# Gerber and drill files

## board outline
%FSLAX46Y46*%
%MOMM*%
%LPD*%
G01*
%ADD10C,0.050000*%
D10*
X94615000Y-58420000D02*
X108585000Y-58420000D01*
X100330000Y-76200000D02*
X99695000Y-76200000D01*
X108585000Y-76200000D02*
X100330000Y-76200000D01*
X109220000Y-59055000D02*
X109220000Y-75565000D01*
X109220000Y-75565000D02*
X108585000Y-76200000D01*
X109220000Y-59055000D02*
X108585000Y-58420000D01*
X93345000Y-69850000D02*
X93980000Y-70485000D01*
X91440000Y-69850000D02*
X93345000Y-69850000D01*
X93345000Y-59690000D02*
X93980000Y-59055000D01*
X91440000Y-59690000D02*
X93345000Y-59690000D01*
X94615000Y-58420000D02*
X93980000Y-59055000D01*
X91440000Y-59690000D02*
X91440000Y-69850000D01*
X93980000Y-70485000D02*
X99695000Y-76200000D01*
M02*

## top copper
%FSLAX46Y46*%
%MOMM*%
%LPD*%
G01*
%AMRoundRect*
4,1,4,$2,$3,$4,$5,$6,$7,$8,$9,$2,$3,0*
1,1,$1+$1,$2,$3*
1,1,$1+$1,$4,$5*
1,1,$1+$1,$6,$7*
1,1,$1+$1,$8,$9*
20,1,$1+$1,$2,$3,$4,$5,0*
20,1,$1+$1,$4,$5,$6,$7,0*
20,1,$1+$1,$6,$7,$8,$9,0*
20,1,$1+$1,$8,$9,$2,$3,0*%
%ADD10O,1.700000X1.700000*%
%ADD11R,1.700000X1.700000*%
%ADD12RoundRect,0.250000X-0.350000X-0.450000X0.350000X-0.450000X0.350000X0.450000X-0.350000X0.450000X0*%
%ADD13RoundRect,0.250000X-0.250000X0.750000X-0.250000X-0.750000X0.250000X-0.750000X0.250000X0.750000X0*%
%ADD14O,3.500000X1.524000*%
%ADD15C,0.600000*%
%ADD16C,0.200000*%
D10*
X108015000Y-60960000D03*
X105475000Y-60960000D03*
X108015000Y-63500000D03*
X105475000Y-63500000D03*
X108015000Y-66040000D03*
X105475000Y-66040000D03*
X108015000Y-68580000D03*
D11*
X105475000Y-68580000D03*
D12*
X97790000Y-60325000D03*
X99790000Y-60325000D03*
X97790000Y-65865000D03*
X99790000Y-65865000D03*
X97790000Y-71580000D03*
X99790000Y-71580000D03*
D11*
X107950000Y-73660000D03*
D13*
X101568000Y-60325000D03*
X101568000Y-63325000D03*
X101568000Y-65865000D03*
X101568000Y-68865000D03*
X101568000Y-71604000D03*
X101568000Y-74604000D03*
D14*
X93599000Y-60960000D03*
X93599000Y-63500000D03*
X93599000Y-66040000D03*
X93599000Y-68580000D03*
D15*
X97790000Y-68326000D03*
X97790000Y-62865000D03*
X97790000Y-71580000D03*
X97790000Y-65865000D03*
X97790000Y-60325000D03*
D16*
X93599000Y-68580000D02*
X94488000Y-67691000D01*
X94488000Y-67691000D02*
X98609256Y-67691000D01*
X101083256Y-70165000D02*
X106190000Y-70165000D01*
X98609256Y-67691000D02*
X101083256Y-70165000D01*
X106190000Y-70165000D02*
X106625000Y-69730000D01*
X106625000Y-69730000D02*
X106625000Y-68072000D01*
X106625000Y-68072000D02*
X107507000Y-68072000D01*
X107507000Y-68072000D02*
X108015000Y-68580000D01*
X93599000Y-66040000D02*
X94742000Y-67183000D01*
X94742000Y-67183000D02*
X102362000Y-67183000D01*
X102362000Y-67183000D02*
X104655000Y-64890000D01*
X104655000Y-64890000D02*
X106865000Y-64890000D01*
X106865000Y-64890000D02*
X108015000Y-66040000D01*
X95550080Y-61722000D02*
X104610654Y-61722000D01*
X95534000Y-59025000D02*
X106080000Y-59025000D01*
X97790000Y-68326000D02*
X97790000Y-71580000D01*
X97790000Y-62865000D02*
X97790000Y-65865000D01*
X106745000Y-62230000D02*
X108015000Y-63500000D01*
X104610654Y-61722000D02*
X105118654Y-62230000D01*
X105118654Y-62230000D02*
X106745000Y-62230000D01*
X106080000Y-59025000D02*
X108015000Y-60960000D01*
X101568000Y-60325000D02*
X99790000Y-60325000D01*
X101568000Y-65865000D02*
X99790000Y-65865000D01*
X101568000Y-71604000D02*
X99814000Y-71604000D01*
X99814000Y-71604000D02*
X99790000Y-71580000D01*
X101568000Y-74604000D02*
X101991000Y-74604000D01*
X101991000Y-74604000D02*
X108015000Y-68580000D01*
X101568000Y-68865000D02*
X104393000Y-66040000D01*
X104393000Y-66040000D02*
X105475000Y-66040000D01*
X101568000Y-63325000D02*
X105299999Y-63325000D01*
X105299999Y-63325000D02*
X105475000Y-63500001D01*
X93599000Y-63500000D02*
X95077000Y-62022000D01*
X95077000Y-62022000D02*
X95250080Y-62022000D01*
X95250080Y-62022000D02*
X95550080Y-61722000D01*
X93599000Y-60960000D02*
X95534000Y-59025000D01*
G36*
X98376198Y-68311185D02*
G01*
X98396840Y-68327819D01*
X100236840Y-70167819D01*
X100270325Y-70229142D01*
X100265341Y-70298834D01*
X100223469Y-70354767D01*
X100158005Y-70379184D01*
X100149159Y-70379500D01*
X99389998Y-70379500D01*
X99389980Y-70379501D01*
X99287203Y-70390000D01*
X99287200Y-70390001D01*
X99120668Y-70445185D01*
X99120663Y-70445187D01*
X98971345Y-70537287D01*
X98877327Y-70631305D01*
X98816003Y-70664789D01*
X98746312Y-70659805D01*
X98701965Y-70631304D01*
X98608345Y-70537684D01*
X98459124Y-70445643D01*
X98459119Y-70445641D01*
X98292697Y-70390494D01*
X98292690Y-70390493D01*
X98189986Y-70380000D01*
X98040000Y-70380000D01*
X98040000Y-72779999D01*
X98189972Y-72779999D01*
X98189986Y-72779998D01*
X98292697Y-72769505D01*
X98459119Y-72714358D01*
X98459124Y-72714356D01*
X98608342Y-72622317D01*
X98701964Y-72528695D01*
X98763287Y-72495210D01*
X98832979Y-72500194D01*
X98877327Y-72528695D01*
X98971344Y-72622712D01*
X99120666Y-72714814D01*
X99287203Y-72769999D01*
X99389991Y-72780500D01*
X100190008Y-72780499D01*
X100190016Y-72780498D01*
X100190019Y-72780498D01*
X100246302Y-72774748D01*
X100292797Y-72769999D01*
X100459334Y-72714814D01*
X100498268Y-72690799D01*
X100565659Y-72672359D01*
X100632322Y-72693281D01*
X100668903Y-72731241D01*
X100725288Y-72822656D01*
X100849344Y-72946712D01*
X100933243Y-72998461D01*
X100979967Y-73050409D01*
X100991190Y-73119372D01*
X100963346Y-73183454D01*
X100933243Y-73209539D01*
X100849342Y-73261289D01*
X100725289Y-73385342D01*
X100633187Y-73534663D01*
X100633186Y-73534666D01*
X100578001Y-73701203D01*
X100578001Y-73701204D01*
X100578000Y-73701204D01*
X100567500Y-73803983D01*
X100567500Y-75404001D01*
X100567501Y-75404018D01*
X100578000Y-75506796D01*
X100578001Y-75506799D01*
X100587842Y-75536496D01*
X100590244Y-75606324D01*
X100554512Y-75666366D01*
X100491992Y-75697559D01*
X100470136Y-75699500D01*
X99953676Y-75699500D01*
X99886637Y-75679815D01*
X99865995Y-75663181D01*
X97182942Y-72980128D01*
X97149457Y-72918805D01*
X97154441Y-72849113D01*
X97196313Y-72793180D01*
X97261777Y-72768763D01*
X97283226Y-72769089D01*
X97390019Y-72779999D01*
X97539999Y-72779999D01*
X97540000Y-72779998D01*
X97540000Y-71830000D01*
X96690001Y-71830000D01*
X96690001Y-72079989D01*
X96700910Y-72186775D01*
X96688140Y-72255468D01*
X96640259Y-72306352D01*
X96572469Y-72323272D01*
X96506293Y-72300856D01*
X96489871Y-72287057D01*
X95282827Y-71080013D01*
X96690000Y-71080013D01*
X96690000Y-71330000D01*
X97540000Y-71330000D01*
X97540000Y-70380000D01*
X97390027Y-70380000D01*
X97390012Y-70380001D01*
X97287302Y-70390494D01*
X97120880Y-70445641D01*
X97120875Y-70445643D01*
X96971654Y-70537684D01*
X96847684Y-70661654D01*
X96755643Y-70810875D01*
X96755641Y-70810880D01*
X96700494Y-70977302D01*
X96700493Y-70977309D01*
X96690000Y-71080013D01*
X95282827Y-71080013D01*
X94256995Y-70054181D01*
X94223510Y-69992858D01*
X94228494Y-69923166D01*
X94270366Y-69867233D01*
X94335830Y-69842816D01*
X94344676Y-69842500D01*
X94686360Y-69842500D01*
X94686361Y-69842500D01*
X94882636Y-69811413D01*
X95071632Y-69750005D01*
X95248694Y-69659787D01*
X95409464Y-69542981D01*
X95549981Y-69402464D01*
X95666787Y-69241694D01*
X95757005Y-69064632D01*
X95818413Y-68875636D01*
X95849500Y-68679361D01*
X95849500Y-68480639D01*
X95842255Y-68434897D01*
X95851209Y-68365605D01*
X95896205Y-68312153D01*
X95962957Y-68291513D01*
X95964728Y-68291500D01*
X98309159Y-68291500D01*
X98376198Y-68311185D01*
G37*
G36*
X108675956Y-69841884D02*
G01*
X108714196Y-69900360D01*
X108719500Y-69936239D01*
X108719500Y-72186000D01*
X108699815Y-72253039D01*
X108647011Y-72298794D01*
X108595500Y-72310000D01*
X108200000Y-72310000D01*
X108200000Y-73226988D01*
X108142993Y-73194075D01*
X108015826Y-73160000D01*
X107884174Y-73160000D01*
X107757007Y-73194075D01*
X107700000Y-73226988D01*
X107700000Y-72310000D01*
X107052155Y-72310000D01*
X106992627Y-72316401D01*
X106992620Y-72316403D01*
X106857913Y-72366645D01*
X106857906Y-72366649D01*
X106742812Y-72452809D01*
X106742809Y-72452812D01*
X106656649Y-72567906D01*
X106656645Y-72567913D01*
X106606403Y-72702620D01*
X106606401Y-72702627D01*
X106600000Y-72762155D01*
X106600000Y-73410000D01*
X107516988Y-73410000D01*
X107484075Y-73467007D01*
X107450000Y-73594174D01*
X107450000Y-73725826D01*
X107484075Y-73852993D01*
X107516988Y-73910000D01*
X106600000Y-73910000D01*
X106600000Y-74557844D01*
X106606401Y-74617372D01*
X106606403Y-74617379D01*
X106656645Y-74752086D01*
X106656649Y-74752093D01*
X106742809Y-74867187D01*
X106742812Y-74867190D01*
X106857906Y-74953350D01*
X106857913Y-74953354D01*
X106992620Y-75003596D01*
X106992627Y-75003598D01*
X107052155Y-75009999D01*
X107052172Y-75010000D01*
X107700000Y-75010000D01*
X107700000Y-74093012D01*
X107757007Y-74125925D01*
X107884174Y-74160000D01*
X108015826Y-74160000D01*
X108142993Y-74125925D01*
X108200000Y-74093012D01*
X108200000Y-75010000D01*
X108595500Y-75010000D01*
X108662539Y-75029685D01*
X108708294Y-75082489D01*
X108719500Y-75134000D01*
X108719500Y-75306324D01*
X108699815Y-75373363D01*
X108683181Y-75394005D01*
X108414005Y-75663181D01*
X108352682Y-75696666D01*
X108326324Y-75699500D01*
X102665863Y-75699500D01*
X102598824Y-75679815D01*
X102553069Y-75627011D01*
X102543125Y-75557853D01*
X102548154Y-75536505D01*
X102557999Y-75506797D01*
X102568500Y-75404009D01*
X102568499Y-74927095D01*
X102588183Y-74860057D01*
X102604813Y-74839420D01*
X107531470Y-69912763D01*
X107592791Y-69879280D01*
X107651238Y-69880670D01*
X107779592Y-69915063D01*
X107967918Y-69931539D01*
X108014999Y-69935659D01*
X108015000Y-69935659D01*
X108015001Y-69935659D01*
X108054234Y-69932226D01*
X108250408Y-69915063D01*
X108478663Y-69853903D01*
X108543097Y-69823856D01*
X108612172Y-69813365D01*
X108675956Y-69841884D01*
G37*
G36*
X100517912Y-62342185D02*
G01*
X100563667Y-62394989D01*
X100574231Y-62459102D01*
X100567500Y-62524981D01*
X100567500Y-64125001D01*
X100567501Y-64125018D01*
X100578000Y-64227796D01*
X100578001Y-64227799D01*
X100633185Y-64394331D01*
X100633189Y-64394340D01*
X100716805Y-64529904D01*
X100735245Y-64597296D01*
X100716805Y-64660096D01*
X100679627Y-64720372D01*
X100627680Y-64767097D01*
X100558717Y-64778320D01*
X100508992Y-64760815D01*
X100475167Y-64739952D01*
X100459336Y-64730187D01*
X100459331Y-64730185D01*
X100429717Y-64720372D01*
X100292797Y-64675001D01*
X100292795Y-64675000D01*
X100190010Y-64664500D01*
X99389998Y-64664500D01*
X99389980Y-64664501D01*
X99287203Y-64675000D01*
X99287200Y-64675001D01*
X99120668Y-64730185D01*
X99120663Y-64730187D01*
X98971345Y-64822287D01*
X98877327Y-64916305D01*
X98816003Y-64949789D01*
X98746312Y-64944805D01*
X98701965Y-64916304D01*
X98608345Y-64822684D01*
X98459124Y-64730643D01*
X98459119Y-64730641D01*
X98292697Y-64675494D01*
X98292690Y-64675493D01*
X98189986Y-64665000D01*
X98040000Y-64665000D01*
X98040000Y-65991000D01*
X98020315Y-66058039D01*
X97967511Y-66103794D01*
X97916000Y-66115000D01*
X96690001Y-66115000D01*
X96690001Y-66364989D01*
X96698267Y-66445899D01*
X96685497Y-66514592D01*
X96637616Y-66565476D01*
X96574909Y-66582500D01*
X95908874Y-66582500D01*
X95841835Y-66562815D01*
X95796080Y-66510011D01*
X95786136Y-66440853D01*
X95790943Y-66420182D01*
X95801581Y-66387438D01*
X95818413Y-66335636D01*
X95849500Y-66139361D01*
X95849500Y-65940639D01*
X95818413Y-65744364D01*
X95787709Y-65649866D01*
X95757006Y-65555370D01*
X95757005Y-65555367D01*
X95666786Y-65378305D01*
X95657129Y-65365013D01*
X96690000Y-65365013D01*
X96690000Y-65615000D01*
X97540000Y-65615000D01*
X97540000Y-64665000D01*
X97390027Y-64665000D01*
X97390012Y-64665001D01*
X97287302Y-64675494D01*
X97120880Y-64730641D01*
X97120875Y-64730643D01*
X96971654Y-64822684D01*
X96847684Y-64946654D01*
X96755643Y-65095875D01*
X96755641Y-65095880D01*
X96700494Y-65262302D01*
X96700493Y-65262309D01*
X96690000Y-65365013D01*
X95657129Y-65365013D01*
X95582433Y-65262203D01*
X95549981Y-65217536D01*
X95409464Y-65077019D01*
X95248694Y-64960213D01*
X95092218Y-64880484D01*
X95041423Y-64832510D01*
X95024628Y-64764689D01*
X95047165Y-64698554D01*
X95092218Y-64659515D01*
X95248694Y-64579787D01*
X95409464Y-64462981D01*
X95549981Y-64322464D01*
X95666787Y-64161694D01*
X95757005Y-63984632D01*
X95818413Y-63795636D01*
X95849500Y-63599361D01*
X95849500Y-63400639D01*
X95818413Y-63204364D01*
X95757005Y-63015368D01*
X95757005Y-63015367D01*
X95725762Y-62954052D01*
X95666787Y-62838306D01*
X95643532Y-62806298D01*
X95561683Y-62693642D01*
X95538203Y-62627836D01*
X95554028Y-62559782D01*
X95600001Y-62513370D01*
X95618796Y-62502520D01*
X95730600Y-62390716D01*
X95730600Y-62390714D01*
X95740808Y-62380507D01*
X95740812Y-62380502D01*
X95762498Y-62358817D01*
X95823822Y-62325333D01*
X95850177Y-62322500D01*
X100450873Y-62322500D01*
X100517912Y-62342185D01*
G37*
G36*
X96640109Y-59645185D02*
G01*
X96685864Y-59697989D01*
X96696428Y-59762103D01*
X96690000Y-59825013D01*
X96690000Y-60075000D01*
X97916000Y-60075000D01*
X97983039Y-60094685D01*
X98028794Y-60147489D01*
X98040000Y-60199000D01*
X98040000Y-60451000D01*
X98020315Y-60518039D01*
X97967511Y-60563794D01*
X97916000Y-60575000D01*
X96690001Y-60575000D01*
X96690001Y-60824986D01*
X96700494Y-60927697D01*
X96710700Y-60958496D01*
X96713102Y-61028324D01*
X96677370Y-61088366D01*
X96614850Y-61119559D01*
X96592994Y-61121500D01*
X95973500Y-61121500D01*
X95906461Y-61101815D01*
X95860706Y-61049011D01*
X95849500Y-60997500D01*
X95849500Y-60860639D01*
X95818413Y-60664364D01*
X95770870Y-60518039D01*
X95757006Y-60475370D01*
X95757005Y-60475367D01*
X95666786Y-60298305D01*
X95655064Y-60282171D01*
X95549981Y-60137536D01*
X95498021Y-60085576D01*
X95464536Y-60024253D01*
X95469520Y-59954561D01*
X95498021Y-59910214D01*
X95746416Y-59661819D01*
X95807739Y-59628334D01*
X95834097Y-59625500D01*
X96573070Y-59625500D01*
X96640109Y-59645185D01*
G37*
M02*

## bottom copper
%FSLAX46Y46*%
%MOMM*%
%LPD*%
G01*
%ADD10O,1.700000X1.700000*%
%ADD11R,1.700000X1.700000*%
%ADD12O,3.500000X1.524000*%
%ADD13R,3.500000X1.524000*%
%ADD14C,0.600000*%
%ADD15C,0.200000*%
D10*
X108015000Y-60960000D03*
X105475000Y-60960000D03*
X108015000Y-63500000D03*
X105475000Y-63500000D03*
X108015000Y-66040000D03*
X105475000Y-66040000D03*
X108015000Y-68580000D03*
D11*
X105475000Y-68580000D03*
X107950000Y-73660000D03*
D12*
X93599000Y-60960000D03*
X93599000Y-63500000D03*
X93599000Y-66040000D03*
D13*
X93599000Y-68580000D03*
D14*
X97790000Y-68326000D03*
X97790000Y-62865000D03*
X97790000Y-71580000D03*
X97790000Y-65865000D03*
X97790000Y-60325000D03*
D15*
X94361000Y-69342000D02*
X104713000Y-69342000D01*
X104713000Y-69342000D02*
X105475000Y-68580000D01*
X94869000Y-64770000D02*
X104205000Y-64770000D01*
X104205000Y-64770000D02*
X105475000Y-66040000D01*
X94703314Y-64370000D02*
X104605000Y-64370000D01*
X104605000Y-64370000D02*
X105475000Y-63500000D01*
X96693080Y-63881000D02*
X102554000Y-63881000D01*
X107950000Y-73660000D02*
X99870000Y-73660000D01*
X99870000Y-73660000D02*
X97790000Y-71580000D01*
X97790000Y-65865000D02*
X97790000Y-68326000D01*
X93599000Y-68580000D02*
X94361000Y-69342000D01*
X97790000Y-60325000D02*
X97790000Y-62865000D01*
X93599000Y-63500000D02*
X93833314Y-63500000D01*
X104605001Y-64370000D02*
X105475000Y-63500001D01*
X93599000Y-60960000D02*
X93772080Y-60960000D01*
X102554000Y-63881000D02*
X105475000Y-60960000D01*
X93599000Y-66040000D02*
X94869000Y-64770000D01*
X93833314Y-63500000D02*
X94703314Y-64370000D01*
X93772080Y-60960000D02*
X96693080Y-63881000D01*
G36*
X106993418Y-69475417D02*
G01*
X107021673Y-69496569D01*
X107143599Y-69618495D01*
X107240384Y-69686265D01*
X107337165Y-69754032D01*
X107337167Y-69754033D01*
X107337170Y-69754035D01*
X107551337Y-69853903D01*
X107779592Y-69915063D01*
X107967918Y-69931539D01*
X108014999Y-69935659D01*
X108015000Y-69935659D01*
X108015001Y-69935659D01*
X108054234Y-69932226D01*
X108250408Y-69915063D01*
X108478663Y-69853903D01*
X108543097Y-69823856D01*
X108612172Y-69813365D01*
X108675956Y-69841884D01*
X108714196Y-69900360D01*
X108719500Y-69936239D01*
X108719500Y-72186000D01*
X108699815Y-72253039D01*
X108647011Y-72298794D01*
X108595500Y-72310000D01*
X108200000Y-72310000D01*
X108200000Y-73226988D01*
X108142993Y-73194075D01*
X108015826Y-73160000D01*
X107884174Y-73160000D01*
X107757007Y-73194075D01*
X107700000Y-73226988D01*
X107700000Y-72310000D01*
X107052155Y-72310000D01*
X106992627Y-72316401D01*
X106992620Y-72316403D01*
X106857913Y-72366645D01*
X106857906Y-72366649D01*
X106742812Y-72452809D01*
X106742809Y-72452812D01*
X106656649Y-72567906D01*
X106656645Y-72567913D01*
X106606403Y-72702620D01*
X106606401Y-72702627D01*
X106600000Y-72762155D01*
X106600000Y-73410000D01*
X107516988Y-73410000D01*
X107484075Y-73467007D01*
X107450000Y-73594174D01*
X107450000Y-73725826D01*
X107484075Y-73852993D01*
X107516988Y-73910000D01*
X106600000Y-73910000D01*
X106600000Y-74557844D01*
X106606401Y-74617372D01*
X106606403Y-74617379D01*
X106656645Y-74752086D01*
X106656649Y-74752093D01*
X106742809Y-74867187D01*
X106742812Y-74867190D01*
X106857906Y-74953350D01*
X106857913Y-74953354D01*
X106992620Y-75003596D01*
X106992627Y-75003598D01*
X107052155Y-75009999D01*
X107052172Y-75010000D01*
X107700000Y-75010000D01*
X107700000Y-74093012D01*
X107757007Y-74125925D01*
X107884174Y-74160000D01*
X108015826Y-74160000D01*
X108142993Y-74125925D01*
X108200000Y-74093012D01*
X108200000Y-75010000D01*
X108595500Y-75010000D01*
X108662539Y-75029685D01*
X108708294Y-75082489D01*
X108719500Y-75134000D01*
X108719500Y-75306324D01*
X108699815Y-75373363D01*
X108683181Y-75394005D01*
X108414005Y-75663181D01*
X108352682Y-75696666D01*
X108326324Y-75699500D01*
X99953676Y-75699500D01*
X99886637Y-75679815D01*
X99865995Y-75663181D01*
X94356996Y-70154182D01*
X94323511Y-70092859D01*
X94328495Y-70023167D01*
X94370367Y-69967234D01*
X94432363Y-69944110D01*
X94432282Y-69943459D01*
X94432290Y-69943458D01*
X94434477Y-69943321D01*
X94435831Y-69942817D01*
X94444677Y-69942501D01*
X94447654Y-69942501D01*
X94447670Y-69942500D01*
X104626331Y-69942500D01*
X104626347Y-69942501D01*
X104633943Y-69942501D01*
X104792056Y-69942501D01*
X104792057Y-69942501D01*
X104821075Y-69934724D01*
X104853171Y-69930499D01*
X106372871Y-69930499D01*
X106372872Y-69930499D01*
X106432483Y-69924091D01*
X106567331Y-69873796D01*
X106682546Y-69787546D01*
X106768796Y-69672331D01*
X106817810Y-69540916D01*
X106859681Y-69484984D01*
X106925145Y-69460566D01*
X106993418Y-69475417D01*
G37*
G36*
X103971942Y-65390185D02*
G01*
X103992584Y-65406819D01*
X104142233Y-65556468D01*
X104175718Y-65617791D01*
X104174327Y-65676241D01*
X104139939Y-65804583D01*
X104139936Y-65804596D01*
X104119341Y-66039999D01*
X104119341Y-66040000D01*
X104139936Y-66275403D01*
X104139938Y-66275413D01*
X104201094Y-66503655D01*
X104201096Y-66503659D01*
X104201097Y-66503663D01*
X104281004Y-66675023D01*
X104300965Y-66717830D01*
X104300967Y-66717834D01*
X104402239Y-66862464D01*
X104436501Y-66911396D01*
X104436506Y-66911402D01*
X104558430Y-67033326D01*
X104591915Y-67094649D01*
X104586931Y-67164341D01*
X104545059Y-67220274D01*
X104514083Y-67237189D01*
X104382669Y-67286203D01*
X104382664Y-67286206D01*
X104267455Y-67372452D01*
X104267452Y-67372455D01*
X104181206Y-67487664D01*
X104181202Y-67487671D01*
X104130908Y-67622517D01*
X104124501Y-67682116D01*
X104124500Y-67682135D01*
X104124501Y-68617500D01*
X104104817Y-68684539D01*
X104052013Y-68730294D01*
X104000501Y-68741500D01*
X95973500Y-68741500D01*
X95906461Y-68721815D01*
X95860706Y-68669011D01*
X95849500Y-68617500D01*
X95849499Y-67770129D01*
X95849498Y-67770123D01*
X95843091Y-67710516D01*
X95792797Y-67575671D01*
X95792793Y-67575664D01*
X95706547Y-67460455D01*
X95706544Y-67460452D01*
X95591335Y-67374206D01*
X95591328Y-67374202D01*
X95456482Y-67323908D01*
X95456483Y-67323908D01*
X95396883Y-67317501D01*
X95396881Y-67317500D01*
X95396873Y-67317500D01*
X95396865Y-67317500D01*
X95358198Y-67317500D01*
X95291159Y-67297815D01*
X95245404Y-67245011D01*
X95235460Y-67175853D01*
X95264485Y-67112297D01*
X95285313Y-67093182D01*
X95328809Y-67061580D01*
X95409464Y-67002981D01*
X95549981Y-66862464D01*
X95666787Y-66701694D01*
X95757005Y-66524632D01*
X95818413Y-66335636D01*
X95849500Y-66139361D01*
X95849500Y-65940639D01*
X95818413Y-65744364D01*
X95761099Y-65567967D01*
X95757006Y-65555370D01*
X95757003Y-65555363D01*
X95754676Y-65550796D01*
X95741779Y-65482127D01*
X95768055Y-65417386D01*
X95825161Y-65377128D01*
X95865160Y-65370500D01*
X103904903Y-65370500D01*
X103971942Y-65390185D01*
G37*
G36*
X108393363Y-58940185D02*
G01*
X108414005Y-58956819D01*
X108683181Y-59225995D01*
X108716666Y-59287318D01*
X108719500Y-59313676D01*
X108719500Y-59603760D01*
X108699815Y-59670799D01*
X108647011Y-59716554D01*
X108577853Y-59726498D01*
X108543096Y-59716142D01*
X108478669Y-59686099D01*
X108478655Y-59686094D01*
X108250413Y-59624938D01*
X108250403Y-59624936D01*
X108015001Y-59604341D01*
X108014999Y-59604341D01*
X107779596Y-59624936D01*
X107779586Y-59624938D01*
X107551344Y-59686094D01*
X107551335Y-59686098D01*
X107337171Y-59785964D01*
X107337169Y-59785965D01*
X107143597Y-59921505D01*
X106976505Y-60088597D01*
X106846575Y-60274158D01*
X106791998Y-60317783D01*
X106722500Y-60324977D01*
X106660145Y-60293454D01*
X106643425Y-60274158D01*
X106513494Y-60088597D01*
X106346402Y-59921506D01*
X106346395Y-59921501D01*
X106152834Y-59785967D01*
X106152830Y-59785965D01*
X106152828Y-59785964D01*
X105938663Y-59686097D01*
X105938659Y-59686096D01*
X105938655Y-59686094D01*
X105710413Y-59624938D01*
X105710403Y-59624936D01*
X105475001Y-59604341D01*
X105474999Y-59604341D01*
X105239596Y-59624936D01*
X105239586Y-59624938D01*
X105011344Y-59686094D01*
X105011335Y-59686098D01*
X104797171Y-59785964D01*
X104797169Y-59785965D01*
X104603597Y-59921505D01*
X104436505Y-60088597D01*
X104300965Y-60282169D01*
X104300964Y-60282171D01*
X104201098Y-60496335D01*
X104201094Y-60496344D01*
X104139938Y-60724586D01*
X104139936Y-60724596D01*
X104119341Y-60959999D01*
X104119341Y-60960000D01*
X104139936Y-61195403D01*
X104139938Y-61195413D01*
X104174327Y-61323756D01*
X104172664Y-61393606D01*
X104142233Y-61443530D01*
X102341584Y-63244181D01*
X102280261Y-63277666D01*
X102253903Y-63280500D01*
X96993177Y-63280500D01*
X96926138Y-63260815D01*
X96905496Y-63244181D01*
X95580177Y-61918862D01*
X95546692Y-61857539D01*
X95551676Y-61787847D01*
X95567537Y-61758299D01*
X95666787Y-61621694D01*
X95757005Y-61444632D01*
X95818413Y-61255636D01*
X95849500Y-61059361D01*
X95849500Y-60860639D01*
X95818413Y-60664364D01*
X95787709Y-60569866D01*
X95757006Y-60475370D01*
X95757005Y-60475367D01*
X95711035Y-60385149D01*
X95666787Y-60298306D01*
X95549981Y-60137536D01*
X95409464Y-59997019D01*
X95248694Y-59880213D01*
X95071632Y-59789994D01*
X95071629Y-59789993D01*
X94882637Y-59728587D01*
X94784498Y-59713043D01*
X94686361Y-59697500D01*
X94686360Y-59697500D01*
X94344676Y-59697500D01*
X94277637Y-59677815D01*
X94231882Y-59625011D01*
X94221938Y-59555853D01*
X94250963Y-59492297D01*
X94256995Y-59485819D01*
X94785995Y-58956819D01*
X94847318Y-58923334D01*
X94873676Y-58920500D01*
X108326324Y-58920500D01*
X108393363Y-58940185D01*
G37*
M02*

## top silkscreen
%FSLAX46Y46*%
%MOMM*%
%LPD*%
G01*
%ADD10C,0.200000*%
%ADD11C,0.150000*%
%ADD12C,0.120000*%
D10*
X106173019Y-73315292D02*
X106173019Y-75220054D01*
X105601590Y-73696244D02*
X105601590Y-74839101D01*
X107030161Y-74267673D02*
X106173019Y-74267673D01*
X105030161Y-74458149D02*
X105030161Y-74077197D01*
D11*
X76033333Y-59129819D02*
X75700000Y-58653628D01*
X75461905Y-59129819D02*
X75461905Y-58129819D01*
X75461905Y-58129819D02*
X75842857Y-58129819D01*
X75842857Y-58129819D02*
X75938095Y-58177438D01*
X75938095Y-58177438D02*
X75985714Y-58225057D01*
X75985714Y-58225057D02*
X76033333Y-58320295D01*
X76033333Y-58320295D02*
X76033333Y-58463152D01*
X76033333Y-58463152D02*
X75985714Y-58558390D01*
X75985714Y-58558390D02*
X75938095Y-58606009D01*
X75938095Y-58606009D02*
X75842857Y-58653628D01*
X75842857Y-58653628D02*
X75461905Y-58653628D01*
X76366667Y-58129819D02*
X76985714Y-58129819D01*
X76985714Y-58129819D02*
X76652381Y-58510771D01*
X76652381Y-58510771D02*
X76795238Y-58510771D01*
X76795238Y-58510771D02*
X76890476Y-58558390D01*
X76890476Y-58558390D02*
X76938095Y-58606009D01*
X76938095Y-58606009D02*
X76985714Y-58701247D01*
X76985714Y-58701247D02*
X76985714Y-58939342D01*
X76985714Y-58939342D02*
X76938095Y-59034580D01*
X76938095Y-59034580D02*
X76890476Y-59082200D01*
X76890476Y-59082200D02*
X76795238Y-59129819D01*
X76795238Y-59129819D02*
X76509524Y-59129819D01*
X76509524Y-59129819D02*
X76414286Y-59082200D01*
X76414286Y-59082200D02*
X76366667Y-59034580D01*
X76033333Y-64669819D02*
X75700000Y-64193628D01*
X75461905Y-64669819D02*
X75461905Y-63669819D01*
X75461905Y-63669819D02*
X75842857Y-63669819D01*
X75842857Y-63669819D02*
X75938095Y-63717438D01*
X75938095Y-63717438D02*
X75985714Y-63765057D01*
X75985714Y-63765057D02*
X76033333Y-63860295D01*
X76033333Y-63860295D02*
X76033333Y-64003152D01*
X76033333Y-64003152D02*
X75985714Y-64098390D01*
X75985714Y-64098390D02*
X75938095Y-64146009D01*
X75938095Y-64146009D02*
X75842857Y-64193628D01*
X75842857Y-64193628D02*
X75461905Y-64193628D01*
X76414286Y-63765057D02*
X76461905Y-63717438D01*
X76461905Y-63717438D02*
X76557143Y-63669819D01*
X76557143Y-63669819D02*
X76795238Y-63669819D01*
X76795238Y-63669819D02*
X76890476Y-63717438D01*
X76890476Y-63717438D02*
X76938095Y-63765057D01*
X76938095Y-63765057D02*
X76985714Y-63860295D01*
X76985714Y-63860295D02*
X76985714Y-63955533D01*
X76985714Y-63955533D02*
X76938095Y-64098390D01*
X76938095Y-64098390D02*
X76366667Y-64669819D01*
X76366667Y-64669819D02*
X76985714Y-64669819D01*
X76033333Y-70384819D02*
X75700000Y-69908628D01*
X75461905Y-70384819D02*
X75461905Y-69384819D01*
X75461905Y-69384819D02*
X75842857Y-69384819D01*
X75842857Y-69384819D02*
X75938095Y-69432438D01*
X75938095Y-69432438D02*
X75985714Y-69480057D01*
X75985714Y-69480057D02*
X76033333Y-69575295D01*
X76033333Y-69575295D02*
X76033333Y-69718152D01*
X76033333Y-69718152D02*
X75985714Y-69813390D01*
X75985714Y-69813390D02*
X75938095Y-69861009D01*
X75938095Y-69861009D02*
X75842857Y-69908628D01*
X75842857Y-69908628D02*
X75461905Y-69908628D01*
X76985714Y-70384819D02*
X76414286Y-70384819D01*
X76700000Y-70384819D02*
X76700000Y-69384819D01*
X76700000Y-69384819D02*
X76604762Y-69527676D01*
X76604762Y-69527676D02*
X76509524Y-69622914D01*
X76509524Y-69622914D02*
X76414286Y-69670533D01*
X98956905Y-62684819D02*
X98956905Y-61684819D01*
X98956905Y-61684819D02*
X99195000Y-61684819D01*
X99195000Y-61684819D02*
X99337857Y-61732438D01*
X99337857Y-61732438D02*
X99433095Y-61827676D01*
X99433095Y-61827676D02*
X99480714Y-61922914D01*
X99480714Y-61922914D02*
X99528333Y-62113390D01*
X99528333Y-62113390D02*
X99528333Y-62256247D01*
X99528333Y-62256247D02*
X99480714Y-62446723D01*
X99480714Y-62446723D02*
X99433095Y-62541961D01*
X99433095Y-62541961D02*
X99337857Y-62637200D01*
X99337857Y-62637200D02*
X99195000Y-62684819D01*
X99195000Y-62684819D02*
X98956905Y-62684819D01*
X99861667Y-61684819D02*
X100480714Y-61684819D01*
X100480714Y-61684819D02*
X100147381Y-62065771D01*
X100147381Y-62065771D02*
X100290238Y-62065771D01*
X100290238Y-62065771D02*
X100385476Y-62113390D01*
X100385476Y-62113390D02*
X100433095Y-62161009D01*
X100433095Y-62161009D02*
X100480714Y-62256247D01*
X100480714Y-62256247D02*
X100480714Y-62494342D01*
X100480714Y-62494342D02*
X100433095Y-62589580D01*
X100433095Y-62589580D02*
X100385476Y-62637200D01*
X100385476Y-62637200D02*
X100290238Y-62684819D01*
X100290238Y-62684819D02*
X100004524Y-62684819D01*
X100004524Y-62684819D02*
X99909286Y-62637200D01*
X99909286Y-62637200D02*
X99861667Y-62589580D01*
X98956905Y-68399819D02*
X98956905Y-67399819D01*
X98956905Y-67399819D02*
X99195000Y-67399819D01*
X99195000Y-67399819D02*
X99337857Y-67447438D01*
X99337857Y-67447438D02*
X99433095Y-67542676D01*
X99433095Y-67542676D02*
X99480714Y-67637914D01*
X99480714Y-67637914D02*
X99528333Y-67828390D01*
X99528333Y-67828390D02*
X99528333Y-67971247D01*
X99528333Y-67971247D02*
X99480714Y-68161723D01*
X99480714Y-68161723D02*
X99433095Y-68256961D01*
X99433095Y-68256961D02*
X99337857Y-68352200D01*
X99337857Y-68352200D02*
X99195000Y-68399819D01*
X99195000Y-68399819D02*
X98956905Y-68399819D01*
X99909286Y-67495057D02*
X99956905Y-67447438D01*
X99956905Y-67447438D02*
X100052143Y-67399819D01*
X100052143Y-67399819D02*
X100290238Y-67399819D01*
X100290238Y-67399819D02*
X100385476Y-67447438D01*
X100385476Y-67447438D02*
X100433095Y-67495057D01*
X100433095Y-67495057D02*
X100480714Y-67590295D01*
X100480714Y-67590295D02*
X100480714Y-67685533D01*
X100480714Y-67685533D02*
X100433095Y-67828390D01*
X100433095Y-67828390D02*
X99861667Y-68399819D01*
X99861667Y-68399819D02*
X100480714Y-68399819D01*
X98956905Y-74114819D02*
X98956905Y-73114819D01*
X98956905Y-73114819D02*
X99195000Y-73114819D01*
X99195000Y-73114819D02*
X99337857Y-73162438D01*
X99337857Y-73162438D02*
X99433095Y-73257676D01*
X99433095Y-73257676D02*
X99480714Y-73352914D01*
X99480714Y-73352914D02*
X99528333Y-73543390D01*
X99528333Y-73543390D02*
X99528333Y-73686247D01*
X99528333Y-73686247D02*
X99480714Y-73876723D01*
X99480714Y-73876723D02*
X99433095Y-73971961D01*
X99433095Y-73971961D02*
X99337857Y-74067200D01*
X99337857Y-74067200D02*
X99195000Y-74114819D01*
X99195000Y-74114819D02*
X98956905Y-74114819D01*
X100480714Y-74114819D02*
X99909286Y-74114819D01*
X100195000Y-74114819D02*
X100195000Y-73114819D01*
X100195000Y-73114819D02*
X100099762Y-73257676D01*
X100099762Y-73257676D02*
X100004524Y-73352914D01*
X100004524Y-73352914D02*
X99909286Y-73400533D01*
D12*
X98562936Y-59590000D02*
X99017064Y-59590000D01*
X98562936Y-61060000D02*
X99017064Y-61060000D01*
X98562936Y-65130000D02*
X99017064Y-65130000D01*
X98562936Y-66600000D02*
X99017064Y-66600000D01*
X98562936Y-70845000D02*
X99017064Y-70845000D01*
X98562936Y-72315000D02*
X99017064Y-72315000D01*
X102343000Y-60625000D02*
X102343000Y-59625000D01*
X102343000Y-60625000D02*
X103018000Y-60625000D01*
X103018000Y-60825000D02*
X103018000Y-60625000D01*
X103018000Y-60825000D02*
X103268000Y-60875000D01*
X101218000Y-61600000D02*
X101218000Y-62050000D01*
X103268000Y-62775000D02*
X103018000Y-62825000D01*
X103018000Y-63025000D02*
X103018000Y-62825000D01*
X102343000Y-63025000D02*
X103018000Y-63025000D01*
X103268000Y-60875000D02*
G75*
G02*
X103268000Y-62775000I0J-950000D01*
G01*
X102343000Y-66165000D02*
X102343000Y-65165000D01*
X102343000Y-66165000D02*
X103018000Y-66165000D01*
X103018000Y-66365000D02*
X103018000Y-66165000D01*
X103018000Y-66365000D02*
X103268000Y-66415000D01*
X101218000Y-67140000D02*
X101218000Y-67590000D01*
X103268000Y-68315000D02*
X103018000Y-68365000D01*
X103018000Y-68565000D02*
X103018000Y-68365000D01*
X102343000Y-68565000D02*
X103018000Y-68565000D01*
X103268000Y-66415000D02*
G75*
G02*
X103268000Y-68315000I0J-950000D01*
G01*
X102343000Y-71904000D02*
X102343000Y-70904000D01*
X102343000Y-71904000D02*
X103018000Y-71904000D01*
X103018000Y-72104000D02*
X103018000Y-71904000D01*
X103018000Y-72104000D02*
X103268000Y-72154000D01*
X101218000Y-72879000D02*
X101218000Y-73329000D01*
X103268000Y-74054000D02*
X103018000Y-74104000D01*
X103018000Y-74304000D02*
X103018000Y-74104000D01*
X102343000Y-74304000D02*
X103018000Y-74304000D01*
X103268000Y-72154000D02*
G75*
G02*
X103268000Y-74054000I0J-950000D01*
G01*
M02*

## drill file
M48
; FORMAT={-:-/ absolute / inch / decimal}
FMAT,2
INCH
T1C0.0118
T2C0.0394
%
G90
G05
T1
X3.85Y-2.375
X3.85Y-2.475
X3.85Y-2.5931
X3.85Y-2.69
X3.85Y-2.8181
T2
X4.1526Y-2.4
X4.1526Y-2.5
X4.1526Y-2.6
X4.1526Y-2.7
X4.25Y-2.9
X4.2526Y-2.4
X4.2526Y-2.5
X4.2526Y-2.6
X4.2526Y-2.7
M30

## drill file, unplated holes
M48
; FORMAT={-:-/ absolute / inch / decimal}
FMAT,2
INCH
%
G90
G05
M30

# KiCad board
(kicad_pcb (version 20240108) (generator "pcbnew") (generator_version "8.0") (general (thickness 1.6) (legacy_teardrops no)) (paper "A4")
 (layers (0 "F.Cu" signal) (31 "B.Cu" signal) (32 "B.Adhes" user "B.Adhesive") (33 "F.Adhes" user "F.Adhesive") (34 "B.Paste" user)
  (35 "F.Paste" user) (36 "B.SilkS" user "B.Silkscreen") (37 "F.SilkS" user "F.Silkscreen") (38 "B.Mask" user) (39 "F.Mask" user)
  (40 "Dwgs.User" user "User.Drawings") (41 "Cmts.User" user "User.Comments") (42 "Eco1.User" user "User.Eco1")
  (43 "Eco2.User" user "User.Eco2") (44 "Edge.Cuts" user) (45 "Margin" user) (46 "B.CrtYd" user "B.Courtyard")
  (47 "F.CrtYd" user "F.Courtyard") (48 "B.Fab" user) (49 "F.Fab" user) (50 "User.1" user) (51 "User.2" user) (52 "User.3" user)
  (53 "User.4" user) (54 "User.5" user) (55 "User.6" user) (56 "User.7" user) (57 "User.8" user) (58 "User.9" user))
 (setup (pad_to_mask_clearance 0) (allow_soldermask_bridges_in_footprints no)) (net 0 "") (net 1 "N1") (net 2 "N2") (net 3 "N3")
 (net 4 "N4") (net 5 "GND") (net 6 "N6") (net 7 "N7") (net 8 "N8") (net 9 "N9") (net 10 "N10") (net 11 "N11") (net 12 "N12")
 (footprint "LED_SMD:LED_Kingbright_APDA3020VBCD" (layer "F.Cu") (at 101.568 67.365 -90)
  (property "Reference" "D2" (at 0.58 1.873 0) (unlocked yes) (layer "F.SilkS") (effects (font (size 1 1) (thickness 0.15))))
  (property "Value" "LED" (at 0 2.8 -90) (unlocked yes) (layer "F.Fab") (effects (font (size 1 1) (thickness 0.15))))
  (fp_line (start -0.225 0.35) (end 0.225 0.35) (stroke (width 0.12) (type solid)) (layer "F.SilkS"))
  (fp_line (start -1.2 -0.775) (end -2.2 -0.775) (stroke (width 0.12) (type solid)) (layer "F.SilkS"))
  (fp_line (start -1.2 -0.775) (end -1.2 -1.45) (stroke (width 0.12) (type solid)) (layer "F.SilkS"))
  (fp_line (start 1.2 -0.775) (end 1.2 -1.45) (stroke (width 0.12) (type solid)) (layer "F.SilkS"))
  (fp_line (start -1 -1.45) (end -1.2 -1.45) (stroke (width 0.12) (type solid)) (layer "F.SilkS"))
  (fp_line (start -1 -1.45) (end -0.95 -1.7) (stroke (width 0.12) (type solid)) (layer "F.SilkS"))
  (fp_line (start 1.2 -1.45) (end 1 -1.45) (stroke (width 0.12) (type solid)) (layer "F.SilkS"))
  (fp_line (start 0.95 -1.7) (end 1 -1.45) (stroke (width 0.12) (type solid)) (layer "F.SilkS"))
  (fp_arc (start -0.95 -1.7) (mid 0 -2.65) (end 0.95 -1.7) (stroke (width 0.12) (type solid)) (layer "F.SilkS"))
  (pad "1" smd roundrect (at -1.5 0 270) (size 2 1) (layers "F.Cu" "F.Paste" "F.Mask") (roundrect_rratio 0.25) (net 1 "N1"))
  (pad "2" smd roundrect (at 1.5 0 270) (size 2 1) (layers "F.Cu" "F.Paste" "F.Mask") (roundrect_rratio 0.25) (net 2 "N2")))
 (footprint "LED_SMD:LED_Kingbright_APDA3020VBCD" (layer "F.Cu") (at 101.568 73.104 -90)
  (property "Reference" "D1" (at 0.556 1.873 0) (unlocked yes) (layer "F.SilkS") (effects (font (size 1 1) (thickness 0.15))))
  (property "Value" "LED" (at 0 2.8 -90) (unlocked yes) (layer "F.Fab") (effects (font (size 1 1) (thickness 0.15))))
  (fp_line (start -0.225 0.35) (end 0.225 0.35) (stroke (width 0.12) (type solid)) (layer "F.SilkS"))
  (fp_line (start -1.2 -0.775) (end -2.2 -0.775) (stroke (width 0.12) (type solid)) (layer "F.SilkS"))
  (fp_line (start -1.2 -0.775) (end -1.2 -1.45) (stroke (width 0.12) (type solid)) (layer "F.SilkS"))
  (fp_line (start 1.2 -0.775) (end 1.2 -1.45) (stroke (width 0.12) (type solid)) (layer "F.SilkS"))
  (fp_line (start -1 -1.45) (end -1.2 -1.45) (stroke (width 0.12) (type solid)) (layer "F.SilkS"))
  (fp_line (start -1 -1.45) (end -0.95 -1.7) (stroke (width 0.12) (type solid)) (layer "F.SilkS"))
  (fp_line (start 1.2 -1.45) (end 1 -1.45) (stroke (width 0.12) (type solid)) (layer "F.SilkS"))
  (fp_line (start 0.95 -1.7) (end 1 -1.45) (stroke (width 0.12) (type solid)) (layer "F.SilkS"))
  (fp_arc (start -0.95 -1.7) (mid 0 -2.65) (end 0.95 -1.7) (stroke (width 0.12) (type solid)) (layer "F.SilkS"))
  (pad "1" smd roundrect (at -1.5 0 270) (size 2 1) (layers "F.Cu" "F.Paste" "F.Mask") (roundrect_rratio 0.25) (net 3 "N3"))
  (pad "2" smd roundrect (at 1.5 0 270) (size 2 1) (layers "F.Cu" "F.Paste" "F.Mask") (roundrect_rratio 0.25) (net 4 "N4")))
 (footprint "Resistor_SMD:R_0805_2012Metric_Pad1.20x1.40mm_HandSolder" (layer "F.Cu") (at 98.79 65.865)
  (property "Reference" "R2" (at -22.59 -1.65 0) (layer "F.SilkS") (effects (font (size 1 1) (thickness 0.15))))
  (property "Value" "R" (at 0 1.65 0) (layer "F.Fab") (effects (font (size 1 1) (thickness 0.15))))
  (fp_line (start -0.227064 -0.735) (end 0.227064 -0.735) (stroke (width 0.12) (type solid)) (layer "F.SilkS"))
  (fp_line (start -0.227064 0.735) (end 0.227064 0.735) (stroke (width 0.12) (type solid)) (layer "F.SilkS"))
  (pad "1" smd roundrect (at -1 0) (size 1.2 1.4) (layers "F.Cu" "F.Paste" "F.Mask") (roundrect_rratio 0.208333) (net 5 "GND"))
  (pad "2" smd roundrect (at 1 0) (size 1.2 1.4) (layers "F.Cu" "F.Paste" "F.Mask") (roundrect_rratio 0.208333) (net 1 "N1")))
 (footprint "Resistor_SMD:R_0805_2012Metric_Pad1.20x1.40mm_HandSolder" (layer "F.Cu") (at 98.79 60.325)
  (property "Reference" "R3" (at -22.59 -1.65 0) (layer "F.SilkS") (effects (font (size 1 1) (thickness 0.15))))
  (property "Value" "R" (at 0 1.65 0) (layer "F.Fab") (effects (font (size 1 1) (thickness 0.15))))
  (fp_line (start -0.227064 -0.735) (end 0.227064 -0.735) (stroke (width 0.12) (type solid)) (layer "F.SilkS"))
  (fp_line (start -0.227064 0.735) (end 0.227064 0.735) (stroke (width 0.12) (type solid)) (layer "F.SilkS"))
  (pad "1" smd roundrect (at -1 0) (size 1.2 1.4) (layers "F.Cu" "F.Paste" "F.Mask") (roundrect_rratio 0.208333) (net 5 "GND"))
  (pad "2" smd roundrect (at 1 0) (size 1.2 1.4) (layers "F.Cu" "F.Paste" "F.Mask") (roundrect_rratio 0.208333) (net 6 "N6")))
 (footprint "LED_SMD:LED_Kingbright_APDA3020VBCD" (layer "F.Cu") (at 101.568 61.825 -90)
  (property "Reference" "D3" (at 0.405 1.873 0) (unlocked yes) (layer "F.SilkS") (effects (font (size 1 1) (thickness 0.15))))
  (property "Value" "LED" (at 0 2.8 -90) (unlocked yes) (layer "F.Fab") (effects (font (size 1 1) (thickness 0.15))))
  (fp_line (start -0.225 0.35) (end 0.225 0.35) (stroke (width 0.12) (type solid)) (layer "F.SilkS"))
  (fp_line (start -1.2 -0.775) (end -2.2 -0.775) (stroke (width 0.12) (type solid)) (layer "F.SilkS"))
  (fp_line (start -1.2 -0.775) (end -1.2 -1.45) (stroke (width 0.12) (type solid)) (layer "F.SilkS"))
  (fp_line (start 1.2 -0.775) (end 1.2 -1.45) (stroke (width 0.12) (type solid)) (layer "F.SilkS"))
  (fp_line (start -1 -1.45) (end -1.2 -1.45) (stroke (width 0.12) (type solid)) (layer "F.SilkS"))
  (fp_line (start -1 -1.45) (end -0.95 -1.7) (stroke (width 0.12) (type solid)) (layer "F.SilkS"))
  (fp_line (start 1.2 -1.45) (end 1 -1.45) (stroke (width 0.12) (type solid)) (layer "F.SilkS"))
  (fp_line (start 0.95 -1.7) (end 1 -1.45) (stroke (width 0.12) (type solid)) (layer "F.SilkS"))
  (fp_arc (start -0.95 -1.7) (mid 0 -2.65) (end 0.95 -1.7) (stroke (width 0.12) (type solid)) (layer "F.SilkS"))
  (pad "1" smd roundrect (at -1.5 0 270) (size 2 1) (layers "F.Cu" "F.Paste" "F.Mask") (roundrect_rratio 0.25) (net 6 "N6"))
  (pad "2" smd roundrect (at 1.5 0 270) (size 2 1) (layers "F.Cu" "F.Paste" "F.Mask") (roundrect_rratio 0.25) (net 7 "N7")))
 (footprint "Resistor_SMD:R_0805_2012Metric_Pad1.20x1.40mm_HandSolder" (layer "F.Cu") (at 98.79 71.58)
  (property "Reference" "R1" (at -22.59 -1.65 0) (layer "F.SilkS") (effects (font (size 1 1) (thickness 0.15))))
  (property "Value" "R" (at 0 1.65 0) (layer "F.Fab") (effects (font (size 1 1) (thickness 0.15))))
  (fp_line (start -0.227064 -0.735) (end 0.227064 -0.735) (stroke (width 0.12) (type solid)) (layer "F.SilkS"))
  (fp_line (start -0.227064 0.735) (end 0.227064 0.735) (stroke (width 0.12) (type solid)) (layer "F.SilkS"))
  (pad "1" smd roundrect (at -1 0) (size 1.2 1.4) (layers "F.Cu" "F.Paste" "F.Mask") (roundrect_rratio 0.208333) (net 5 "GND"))
  (pad "2" smd roundrect (at 1 0) (size 1.2 1.4) (layers "F.Cu" "F.Paste" "F.Mask") (roundrect_rratio 0.208333) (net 3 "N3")))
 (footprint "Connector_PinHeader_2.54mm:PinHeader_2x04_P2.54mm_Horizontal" (layer "B.Cu") (at 105.475 68.58)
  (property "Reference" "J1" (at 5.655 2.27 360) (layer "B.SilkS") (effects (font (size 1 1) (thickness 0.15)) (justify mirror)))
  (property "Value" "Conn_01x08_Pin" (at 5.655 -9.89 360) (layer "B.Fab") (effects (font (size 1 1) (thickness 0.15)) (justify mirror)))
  (pad "1" thru_hole rect (at 0 0) (size 1.7 1.7) (drill 1) (layers "*.Cu" "*.Mask") (remove_unused_layers no) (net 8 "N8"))
  (pad "2" thru_hole oval (at 2.54 0) (size 1.7 1.7) (drill 1) (layers "*.Cu" "*.Mask") (remove_unused_layers no) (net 4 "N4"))
  (pad "3" thru_hole oval (at 0 -2.54) (size 1.7 1.7) (drill 1) (layers "*.Cu" "*.Mask") (remove_unused_layers no) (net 2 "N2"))
  (pad "4" thru_hole oval (at 2.54 -2.54) (size 1.7 1.7) (drill 1) (layers "*.Cu" "*.Mask") (remove_unused_layers no) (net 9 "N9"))
  (pad "5" thru_hole oval (at 0 -5.08) (size 1.7 1.7) (drill 1) (layers "*.Cu" "*.Mask") (remove_unused_layers no) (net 7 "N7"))
  (pad "6" thru_hole oval (at 2.54 -5.08) (size 1.7 1.7) (drill 1) (layers "*.Cu" "*.Mask") (remove_unused_layers no) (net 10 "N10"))
  (pad "7" thru_hole oval (at 0 -7.62) (size 1.7 1.7) (drill 1) (layers "*.Cu" "*.Mask") (remove_unused_layers no) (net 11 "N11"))
  (pad "8" thru_hole oval (at 2.54 -7.62) (size 1.7 1.7) (drill 1) (layers "*.Cu" "*.Mask") (remove_unused_layers no) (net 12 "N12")))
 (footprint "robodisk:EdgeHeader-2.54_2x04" (layer "B.Cu") (at 91.059 68.58 -90)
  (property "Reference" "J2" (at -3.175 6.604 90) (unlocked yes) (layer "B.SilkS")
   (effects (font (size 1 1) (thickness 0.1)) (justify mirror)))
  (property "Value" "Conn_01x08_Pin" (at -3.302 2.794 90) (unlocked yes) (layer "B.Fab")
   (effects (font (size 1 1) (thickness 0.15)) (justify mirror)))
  (pad "1" smd rect (at 0 -2.54 180) (size 3.5 1.524) (layers "B.Cu" "B.Paste" "B.Mask") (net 8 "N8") (thermal_bridge_angle 45))
  (pad "2" smd oval (at 0 -2.54) (size 3.5 1.524) (layers "F.Cu" "F.Paste" "F.Mask") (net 4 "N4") (thermal_bridge_angle 45))
  (pad "3" smd oval (at -2.54 -2.54 180) (size 3.5 1.524) (layers "B.Cu" "B.Paste" "B.Mask") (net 2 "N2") (thermal_bridge_angle 45))
  (pad "4" smd oval (at -2.54 -2.54) (size 3.5 1.524) (layers "F.Cu" "F.Paste" "F.Mask") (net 9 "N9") (thermal_bridge_angle 45))
  (pad "5" smd oval (at -5.08 -2.54 180) (size 3.5 1.524) (layers "B.Cu" "B.Paste" "B.Mask") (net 7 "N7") (thermal_bridge_angle 45))
  (pad "6" smd oval (at -5.08 -2.54) (size 3.5 1.524) (layers "F.Cu" "F.Paste" "F.Mask") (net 10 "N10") (thermal_bridge_angle 45))
  (pad "7" smd oval (at -7.62 -2.54 180) (size 3.5 1.524) (layers "B.Cu" "B.Paste" "B.Mask") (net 11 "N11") (thermal_bridge_angle 45))
  (pad "8" smd oval (at -7.62 -2.54) (size 3.5 1.524) (layers "F.Cu" "F.Paste" "F.Mask") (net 12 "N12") (thermal_bridge_angle 45)))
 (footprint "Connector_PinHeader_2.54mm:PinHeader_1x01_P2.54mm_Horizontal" (layer "B.Cu") (at 107.95 73.66)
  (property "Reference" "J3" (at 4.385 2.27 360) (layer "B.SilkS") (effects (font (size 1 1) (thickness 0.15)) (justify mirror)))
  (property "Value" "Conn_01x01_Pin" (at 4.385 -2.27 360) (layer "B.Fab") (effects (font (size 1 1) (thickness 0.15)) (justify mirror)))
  (pad "1" thru_hole rect (at 0 0) (size 1.7 1.7) (drill 1) (layers "*.Cu" "*.Mask") (remove_unused_layers no) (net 5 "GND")))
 (gr_line (start 91.44 59.69) (end 91.44 69.85) (stroke (width 0.05) (type default)) (layer "Edge.Cuts"))
 (gr_line (start 93.98 70.485) (end 99.695 76.2) (stroke (width 0.05) (type default)) (layer "Edge.Cuts"))
 (gr_line (start 109.22 59.055) (end 109.22 75.565) (stroke (width 0.05) (type default)) (layer "Edge.Cuts"))
 (gr_line (start 108.585 76.2) (end 100.33 76.2) (stroke (width 0.05) (type default)) (layer "Edge.Cuts"))
 (gr_line (start 91.44 69.85) (end 93.345 69.85) (stroke (width 0.05) (type default)) (layer "Edge.Cuts"))
 (gr_line (start 109.22 59.055) (end 108.585 58.42) (stroke (width 0.05) (type default)) (layer "Edge.Cuts"))
 (gr_line (start 93.345 69.85) (end 93.98 70.485) (stroke (width 0.05) (type default)) (layer "Edge.Cuts"))
 (gr_line (start 100.33 76.2) (end 99.695 76.2) (stroke (width 0.05) (type default)) (layer "Edge.Cuts"))
 (gr_line (start 94.615 58.42) (end 108.585 58.42) (stroke (width 0.05) (type default)) (layer "Edge.Cuts"))
 (gr_line (start 109.22 75.565) (end 108.585 76.2) (stroke (width 0.05) (type default)) (layer "Edge.Cuts"))
 (gr_line (start 93.345 59.69) (end 93.98 59.055) (stroke (width 0.05) (type default)) (layer "Edge.Cuts"))
 (gr_line (start 91.44 59.69) (end 93.345 59.69) (stroke (width 0.05) (type default)) (layer "Edge.Cuts"))
 (gr_line (start 94.615 58.42) (end 93.98 59.055) (stroke (width 0.05) (type default)) (layer "Edge.Cuts"))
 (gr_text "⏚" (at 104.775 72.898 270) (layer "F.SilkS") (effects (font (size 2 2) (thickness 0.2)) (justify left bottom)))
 (segment (start 97.79 62.865) (end 97.79 65.865) (width 0.2) (layer "F.Cu") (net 5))
 (segment (start 97.79 68.326) (end 97.79 71.58) (width 0.2) (layer "F.Cu") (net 5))
 (via (at 97.79 71.58) (size 0.6) (drill 0.3) (layers "F.Cu" "B.Cu") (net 5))
 (via (at 97.79 62.865) (size 0.6) (drill 0.3) (layers "F.Cu" "B.Cu") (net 5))
 (via (at 97.79 68.326) (size 0.6) (drill 0.3) (layers "F.Cu" "B.Cu") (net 5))
 (via (at 97.79 65.865) (size 0.6) (drill 0.3) (layers "F.Cu" "B.Cu") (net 5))
 (via (at 97.79 60.325) (size 0.6) (drill 0.3) (layers "F.Cu" "B.Cu") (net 5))
 (segment (start 99.87 73.66) (end 97.79 71.58) (width 0.2) (layer "B.Cu") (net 5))
 (segment (start 97.79 60.325) (end 97.79 62.865) (width 0.2) (layer "B.Cu") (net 5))
 (segment (start 97.79 65.865) (end 97.79 68.326) (width 0.2) (layer "B.Cu") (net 5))
 (segment (start 107.95 73.66) (end 99.87 73.66) (width 0.2) (layer "B.Cu") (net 5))
 (segment (start 106.625 68.072) (end 107.507 68.072) (width 0.2) (layer "F.Cu") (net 4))
 (segment (start 106.19 70.165) (end 106.625 69.73) (width 0.2) (layer "F.Cu") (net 4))
 (segment (start 93.599 68.58) (end 94.488 67.691) (width 0.2) (layer "F.Cu") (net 4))
 (segment (start 94.488 67.691) (end 98.609256 67.691) (width 0.2) (layer "F.Cu") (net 4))
 (segment (start 107.507 68.072) (end 108.015 68.58) (width 0.2) (layer "F.Cu") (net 4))
 (segment (start 101.991 74.604) (end 108.015 68.58) (width 0.2) (layer "F.Cu") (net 4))
 (segment (start 101.568 74.604) (end 101.991 74.604) (width 0.2) (layer "F.Cu") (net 4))
 (segment (start 101.083256 70.165) (end 106.19 70.165) (width 0.2) (layer "F.Cu") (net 4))
 (segment (start 106.625 69.73) (end 106.625 68.072) (width 0.2) (layer "F.Cu") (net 4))
 (segment (start 98.609256 67.691) (end 101.083256 70.165) (width 0.2) (layer "F.Cu") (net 4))
 (segment (start 101.568 68.865) (end 104.393 66.04) (width 0.2) (layer "F.Cu") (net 2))
 (segment (start 104.393 66.04) (end 105.475 66.04) (width 0.2) (layer "F.Cu") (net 2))
 (segment (start 93.599 66.04) (end 94.869 64.77) (width 0.2) (layer "B.Cu") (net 2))
 (segment (start 94.869 64.77) (end 104.205 64.77) (width 0.2) (layer "B.Cu") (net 2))
 (segment (start 104.205 64.77) (end 105.475 66.04) (width 0.2) (layer "B.Cu") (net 2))
 (segment (start 105.299999 63.325) (end 105.475 63.500001) (width 0.2) (layer "F.Cu") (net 7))
 (segment (start 101.568 63.325) (end 105.299999 63.325) (width 0.2) (layer "F.Cu") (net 7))
 (segment (start 104.605 64.37) (end 105.475 63.5) (width 0.2) (layer "B.Cu") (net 7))
 (segment (start 93.599 63.5) (end 93.833314 63.5) (width 0.2) (layer "B.Cu") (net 7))
 (segment (start 94.703314 64.37) (end 104.605 64.37) (width 0.2) (layer "B.Cu") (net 7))
 (segment (start 104.605001 64.37) (end 105.475 63.500001) (width 0.2) (layer "B.Cu") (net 7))
 (segment (start 93.833314 63.5) (end 94.703314 64.37) (width 0.2) (layer "B.Cu") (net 7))
 (segment (start 94.361 69.342) (end 104.713 69.342) (width 0.2) (layer "B.Cu") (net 8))
 (segment (start 104.713 69.342) (end 105.475 68.58) (width 0.2) (layer "B.Cu") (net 8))
 (segment (start 93.599 68.58) (end 94.361 69.342) (width 0.2) (layer "B.Cu") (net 8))
 (segment (start 95.077 62.022) (end 95.25008 62.022) (width 0.2) (layer "F.Cu") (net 10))
 (segment (start 106.745 62.23) (end 108.015 63.5) (width 0.2) (layer "F.Cu") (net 10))
 (segment (start 93.599 63.5) (end 95.077 62.022) (width 0.2) (layer "F.Cu") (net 10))
 (segment (start 104.610654 61.722) (end 105.118654 62.23) (width 0.2) (layer "F.Cu") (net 10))
 (segment (start 105.118654 62.23) (end 106.745 62.23) (width 0.2) (layer "F.Cu") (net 10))
 (segment (start 95.55008 61.722) (end 104.610654 61.722) (width 0.2) (layer "F.Cu") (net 10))
 (segment (start 95.25008 62.022) (end 95.55008 61.722) (width 0.2) (layer "F.Cu") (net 10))
 (segment (start 93.599 60.96) (end 95.534 59.025) (width 0.2) (layer "F.Cu") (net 12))
 (segment (start 95.534 59.025) (end 106.08 59.025) (width 0.2) (layer "F.Cu") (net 12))
 (segment (start 106.08 59.025) (end 108.015 60.96) (width 0.2) (layer "F.Cu") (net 12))
 (segment (start 93.599 66.04) (end 94.742 67.183) (width 0.2) (layer "F.Cu") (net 9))
 (segment (start 102.362 67.183) (end 104.655 64.89) (width 0.2) (layer "F.Cu") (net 9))
 (segment (start 104.655 64.89) (end 106.865 64.89) (width 0.2) (layer "F.Cu") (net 9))
 (segment (start 94.742 67.183) (end 102.362 67.183) (width 0.2) (layer "F.Cu") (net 9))
 (segment (start 106.865 64.89) (end 108.015 66.04) (width 0.2) (layer "F.Cu") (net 9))
 (segment (start 93.599 60.96) (end 93.77208 60.96) (width 0.2) (layer "B.Cu") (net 11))
 (segment (start 96.69308 63.881) (end 102.554 63.881) (width 0.2) (layer "B.Cu") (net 11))
 (segment (start 93.77208 60.96) (end 96.69308 63.881) (width 0.2) (layer "B.Cu") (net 11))
 (segment (start 102.554 63.881) (end 105.475 60.96) (width 0.2) (layer "B.Cu") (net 11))
 (segment (start 99.814 71.604) (end 99.79 71.58) (width 0.2) (layer "F.Cu") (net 3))
 (segment (start 101.568 71.604) (end 99.814 71.604) (width 0.2) (layer "F.Cu") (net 3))
 (segment (start 101.568 65.865) (end 99.79 65.865) (width 0.2) (layer "F.Cu") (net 1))
 (segment (start 101.568 60.325) (end 99.79 60.325) (width 0.2) (layer "F.Cu") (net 6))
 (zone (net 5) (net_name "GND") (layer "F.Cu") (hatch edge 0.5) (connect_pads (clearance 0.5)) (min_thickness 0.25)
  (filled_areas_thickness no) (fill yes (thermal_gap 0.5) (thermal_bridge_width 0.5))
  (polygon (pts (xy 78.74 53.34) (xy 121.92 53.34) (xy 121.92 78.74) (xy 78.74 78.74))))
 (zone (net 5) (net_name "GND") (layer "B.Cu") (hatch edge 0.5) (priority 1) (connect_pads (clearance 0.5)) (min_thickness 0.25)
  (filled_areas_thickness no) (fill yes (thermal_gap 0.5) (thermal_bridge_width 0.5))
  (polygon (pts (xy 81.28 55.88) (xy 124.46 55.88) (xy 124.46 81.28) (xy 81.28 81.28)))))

